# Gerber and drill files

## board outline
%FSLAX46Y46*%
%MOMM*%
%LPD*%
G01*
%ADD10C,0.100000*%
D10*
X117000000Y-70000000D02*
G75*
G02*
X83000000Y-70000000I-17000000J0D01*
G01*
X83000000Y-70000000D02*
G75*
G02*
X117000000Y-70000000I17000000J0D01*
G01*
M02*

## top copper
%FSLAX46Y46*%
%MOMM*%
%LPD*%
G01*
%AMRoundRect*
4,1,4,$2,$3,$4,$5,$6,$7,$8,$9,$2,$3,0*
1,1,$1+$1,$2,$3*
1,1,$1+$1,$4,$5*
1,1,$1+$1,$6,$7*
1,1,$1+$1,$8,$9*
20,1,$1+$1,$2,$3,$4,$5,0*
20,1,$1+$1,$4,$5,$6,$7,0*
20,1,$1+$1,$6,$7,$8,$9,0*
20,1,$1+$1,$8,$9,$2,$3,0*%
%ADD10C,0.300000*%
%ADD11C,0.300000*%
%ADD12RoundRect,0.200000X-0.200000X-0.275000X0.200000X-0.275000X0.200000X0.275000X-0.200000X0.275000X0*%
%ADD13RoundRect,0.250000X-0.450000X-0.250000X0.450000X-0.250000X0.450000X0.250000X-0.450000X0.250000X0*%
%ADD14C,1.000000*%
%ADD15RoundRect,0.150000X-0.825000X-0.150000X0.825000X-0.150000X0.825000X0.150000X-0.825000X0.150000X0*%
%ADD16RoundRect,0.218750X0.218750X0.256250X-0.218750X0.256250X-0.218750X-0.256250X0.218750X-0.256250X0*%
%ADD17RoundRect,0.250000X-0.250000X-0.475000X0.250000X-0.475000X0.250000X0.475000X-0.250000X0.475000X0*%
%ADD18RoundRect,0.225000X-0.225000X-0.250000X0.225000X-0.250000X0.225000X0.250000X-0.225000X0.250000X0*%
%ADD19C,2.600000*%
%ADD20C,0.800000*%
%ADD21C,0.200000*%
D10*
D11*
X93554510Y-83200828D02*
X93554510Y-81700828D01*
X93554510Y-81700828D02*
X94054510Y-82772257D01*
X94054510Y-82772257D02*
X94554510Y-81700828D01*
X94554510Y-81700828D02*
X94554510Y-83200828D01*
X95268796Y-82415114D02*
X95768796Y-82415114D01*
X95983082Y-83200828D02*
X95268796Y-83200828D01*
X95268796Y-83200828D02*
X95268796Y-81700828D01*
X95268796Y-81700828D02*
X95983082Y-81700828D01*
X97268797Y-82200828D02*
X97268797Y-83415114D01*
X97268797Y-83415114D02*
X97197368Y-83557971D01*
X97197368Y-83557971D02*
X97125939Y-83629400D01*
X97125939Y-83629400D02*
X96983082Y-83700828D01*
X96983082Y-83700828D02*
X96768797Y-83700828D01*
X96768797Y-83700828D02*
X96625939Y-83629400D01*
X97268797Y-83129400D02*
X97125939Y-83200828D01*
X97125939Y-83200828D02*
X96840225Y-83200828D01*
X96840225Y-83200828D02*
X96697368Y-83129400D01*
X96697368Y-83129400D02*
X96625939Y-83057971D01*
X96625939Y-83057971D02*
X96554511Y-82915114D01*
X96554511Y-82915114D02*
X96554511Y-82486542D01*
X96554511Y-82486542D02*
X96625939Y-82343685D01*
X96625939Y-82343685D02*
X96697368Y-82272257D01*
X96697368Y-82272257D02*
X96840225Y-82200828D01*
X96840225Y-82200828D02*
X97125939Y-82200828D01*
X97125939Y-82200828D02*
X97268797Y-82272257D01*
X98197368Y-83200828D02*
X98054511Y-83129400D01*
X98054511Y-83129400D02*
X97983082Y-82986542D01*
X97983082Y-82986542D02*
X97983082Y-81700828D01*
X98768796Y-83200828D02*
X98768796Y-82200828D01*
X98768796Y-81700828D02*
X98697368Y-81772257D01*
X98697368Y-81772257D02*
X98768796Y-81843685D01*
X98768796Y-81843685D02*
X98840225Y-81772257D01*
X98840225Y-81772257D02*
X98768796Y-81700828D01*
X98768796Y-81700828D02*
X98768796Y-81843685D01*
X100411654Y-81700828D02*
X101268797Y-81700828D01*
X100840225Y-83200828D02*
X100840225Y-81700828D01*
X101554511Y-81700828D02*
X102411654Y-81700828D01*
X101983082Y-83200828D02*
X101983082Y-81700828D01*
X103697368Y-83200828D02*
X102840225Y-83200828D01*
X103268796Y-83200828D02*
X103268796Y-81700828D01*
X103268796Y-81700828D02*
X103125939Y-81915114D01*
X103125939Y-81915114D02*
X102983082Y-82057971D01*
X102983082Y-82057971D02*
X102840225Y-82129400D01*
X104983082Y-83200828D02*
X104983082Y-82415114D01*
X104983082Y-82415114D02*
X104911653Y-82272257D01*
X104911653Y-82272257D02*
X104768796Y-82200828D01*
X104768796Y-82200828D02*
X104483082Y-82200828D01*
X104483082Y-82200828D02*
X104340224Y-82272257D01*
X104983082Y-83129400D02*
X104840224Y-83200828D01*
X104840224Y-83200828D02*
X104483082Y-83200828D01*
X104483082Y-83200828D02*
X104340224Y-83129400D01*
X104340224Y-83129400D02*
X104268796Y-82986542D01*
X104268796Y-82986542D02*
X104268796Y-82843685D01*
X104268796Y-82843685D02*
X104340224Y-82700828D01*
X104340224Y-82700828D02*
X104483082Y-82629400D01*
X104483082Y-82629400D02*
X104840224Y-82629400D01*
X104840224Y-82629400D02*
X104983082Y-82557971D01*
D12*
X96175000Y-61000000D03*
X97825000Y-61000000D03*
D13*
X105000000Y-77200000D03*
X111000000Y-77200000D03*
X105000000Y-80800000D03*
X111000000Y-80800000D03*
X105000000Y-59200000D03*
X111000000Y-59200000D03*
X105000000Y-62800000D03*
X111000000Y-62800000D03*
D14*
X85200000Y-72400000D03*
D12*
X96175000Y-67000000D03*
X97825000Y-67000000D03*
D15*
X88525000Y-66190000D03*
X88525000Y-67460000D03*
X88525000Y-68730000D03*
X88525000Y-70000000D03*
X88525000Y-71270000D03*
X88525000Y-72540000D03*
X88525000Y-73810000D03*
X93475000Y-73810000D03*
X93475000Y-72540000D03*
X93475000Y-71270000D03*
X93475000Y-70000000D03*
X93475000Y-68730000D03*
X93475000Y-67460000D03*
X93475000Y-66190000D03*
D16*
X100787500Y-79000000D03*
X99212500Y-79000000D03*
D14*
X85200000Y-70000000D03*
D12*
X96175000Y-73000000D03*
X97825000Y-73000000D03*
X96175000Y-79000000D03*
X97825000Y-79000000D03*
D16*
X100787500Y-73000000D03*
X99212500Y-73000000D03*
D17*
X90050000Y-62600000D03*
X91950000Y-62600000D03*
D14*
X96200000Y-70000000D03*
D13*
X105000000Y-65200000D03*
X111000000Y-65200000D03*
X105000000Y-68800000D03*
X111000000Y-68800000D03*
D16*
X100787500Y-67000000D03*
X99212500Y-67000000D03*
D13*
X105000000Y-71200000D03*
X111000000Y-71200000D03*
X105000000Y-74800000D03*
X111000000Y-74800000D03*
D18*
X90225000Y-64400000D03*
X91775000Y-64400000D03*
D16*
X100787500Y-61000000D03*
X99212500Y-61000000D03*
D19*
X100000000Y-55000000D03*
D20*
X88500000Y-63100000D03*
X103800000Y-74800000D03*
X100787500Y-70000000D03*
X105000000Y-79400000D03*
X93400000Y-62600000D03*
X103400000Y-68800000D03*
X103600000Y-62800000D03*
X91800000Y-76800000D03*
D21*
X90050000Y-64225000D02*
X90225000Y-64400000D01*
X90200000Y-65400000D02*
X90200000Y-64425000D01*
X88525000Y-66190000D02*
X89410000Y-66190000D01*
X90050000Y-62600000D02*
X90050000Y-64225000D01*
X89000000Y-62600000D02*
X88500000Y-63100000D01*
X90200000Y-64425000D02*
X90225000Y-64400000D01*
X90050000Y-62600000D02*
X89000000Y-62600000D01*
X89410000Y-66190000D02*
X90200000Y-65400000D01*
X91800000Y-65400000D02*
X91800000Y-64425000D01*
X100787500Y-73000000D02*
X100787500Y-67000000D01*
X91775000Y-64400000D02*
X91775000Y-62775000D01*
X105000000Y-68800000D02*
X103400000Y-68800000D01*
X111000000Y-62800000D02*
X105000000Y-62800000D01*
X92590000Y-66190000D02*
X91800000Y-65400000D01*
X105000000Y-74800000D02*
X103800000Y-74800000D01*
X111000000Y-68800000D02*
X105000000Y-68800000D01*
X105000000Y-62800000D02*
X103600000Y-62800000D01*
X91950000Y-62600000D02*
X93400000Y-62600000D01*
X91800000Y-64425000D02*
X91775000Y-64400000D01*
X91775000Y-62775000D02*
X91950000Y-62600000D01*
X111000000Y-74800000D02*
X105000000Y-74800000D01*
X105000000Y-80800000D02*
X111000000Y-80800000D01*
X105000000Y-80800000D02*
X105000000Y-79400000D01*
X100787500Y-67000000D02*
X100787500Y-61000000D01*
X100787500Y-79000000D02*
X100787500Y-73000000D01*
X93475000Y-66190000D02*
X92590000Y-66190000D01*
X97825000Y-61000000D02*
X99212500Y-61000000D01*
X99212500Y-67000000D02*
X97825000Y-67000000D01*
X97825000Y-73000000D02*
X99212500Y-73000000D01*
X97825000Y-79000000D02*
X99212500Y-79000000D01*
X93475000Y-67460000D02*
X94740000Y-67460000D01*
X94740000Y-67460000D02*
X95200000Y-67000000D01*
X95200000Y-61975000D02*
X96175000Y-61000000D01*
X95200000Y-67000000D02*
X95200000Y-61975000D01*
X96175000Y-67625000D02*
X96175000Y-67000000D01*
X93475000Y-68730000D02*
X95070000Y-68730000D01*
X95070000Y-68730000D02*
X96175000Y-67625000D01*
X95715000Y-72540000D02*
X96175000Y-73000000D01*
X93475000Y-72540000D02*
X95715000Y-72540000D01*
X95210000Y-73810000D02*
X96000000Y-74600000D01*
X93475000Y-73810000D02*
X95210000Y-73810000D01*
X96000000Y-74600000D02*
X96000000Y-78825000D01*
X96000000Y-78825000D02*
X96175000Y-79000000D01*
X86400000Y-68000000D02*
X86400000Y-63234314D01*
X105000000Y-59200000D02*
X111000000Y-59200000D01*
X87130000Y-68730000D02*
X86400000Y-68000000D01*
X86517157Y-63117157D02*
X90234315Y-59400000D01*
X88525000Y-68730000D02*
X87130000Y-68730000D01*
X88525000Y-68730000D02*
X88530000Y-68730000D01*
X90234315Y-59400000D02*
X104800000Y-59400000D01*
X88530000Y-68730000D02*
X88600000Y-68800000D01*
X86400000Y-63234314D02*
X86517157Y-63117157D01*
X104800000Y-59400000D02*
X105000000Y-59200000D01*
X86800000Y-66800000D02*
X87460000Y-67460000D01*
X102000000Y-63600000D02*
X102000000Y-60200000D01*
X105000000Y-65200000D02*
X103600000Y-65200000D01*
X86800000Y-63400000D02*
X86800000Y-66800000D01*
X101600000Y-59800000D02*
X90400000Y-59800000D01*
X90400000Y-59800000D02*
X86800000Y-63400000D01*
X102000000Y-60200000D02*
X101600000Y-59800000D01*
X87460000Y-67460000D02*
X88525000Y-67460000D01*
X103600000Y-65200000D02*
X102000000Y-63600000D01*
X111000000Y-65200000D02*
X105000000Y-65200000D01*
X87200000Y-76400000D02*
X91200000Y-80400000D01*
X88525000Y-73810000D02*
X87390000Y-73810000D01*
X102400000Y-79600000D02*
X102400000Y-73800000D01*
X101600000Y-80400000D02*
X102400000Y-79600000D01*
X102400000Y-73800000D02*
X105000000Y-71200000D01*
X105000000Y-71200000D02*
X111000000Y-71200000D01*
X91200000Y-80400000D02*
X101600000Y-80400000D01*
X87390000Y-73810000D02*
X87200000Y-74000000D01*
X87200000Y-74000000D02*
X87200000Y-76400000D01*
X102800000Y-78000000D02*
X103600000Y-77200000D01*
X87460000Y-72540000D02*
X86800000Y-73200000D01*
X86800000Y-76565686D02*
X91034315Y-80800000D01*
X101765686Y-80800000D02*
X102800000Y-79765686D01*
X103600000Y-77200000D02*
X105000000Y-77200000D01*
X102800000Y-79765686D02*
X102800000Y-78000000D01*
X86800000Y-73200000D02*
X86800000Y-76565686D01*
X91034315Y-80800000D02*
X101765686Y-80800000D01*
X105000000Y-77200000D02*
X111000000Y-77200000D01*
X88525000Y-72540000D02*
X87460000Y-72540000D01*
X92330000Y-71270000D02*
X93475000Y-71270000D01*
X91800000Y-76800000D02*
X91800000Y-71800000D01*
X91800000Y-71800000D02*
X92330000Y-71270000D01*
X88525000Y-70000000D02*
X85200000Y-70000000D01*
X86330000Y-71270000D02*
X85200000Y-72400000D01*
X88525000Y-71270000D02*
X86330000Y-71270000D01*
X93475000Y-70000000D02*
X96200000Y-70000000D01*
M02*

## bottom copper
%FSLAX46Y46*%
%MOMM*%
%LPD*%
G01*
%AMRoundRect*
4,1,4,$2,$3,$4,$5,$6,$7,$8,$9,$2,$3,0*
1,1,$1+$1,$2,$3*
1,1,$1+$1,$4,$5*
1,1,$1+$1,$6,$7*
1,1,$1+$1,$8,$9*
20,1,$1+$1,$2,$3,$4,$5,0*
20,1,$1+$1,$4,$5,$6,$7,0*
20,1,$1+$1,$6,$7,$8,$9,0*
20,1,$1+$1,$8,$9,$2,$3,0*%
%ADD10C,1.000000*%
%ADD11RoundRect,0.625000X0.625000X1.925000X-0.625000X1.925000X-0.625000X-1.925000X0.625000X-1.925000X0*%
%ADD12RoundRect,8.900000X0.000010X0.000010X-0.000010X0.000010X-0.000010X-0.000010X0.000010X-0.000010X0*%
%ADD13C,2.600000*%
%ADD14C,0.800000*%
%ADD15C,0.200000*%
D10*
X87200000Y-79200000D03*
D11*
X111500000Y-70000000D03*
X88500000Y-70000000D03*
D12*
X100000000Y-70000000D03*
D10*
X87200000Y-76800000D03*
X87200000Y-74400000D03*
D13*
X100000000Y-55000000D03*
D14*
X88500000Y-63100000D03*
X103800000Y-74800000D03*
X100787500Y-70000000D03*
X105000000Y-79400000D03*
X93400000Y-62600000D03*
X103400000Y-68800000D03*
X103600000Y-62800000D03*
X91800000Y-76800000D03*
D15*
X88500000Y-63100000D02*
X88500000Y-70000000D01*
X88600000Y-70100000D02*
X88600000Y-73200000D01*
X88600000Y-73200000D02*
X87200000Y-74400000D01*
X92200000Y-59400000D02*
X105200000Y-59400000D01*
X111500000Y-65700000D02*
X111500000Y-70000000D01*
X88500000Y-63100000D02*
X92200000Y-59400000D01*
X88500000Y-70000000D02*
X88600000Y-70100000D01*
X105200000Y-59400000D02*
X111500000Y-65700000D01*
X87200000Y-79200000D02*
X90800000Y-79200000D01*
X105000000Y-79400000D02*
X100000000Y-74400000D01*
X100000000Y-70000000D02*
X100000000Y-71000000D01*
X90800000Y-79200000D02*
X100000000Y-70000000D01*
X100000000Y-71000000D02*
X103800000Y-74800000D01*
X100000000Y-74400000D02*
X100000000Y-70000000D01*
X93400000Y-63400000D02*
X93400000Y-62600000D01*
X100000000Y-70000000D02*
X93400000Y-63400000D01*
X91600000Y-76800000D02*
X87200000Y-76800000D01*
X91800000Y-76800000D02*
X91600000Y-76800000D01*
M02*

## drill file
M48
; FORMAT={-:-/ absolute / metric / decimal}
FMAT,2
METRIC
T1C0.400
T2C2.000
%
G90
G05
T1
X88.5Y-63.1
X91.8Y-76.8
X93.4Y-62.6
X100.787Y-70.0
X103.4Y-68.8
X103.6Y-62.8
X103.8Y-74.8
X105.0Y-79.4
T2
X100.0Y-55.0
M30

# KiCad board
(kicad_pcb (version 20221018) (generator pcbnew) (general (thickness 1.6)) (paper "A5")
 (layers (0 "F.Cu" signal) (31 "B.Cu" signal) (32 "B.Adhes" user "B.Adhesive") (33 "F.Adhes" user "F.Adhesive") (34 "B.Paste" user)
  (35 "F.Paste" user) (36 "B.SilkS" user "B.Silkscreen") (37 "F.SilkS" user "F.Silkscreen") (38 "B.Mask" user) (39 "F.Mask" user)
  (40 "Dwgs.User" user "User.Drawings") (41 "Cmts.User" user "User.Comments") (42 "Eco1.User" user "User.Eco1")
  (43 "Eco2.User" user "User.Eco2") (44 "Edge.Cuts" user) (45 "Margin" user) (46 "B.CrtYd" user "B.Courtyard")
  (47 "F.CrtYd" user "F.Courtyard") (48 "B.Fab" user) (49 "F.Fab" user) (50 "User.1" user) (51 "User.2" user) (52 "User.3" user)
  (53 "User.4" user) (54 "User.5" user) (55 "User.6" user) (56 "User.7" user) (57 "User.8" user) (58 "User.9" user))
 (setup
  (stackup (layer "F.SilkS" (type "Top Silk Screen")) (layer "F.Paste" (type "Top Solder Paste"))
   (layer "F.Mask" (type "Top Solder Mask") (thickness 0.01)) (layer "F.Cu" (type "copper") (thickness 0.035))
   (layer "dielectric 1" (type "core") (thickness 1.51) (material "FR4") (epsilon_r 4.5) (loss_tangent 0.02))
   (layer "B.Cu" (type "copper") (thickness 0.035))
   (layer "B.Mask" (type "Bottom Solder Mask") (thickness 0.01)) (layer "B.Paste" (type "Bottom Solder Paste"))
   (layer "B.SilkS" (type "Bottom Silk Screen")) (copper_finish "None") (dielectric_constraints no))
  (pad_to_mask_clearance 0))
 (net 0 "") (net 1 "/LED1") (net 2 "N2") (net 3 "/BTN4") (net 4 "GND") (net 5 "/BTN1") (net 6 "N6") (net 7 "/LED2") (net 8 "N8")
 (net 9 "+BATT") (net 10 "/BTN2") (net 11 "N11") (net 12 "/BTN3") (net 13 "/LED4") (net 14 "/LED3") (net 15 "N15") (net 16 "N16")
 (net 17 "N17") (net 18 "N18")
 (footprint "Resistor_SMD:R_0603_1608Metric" (layer "F.Cu") (at 97 61)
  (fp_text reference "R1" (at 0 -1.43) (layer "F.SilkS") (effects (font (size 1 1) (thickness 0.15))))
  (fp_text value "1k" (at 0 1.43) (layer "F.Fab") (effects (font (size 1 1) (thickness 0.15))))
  (pad "1" smd roundrect (at -0.825 0) (size 0.8 0.95) (layers "F.Cu" "F.Paste" "F.Mask") (roundrect_rratio 0.25) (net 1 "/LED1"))
  (pad "2" smd roundrect (at 0.825 0) (size 0.8 0.95) (layers "F.Cu" "F.Paste" "F.Mask") (roundrect_rratio 0.25) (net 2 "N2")))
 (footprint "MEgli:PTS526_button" (layer "F.Cu") (at 108 79)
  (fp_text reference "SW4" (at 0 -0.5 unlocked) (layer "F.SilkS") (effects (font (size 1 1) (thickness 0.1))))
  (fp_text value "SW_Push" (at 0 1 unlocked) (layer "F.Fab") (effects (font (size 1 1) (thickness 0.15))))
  (pad "1" smd roundrect (at -3 -1.8) (size 1.4 1) (layers "F.Cu" "F.Paste" "F.Mask") (roundrect_rratio 0.25) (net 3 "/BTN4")
   (thermal_bridge_angle 45))
  (pad "1" smd roundrect (at 3 -1.8) (size 1.4 1) (layers "F.Cu" "F.Paste" "F.Mask") (roundrect_rratio 0.25) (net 3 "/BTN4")
   (thermal_bridge_angle 45))
  (pad "2" smd roundrect (at -3 1.8) (size 1.4 1) (layers "F.Cu" "F.Paste" "F.Mask") (roundrect_rratio 0.25) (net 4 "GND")
   (thermal_bridge_angle 45))
  (pad "2" smd roundrect (at 3 1.8) (size 1.4 1) (layers "F.Cu" "F.Paste" "F.Mask") (roundrect_rratio 0.25) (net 4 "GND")
   (thermal_bridge_angle 45)))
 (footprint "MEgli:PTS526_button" (layer "F.Cu") (at 108 61)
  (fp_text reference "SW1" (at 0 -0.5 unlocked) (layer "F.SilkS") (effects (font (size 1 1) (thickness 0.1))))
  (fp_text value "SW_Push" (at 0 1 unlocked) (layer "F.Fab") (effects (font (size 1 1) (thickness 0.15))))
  (pad "1" smd roundrect (at -3 -1.8) (size 1.4 1) (layers "F.Cu" "F.Paste" "F.Mask") (roundrect_rratio 0.25) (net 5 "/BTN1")
   (thermal_bridge_angle 45))
  (pad "1" smd roundrect (at 3 -1.8) (size 1.4 1) (layers "F.Cu" "F.Paste" "F.Mask") (roundrect_rratio 0.25) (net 5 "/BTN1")
   (thermal_bridge_angle 45))
  (pad "2" smd roundrect (at -3 1.8) (size 1.4 1) (layers "F.Cu" "F.Paste" "F.Mask") (roundrect_rratio 0.25) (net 4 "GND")
   (thermal_bridge_angle 45))
  (pad "2" smd roundrect (at 3 1.8) (size 1.4 1) (layers "F.Cu" "F.Paste" "F.Mask") (roundrect_rratio 0.25) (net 4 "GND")
   (thermal_bridge_angle 45)))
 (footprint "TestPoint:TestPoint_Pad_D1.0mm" (layer "F.Cu") (at 85.2 72.4)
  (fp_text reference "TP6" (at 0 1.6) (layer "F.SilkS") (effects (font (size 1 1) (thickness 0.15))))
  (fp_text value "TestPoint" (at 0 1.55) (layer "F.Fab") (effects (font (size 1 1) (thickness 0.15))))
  (pad "1" smd circle (at 0 0) (size 1 1) (layers "F.Cu" "F.Mask") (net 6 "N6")))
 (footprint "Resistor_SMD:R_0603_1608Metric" (layer "F.Cu") (at 97 67)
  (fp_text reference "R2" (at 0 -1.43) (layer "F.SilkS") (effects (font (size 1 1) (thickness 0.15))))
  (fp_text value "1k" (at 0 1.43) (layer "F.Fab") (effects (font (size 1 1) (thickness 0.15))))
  (pad "1" smd roundrect (at -0.825 0) (size 0.8 0.95) (layers "F.Cu" "F.Paste" "F.Mask") (roundrect_rratio 0.25) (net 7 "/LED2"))
  (pad "2" smd roundrect (at 0.825 0) (size 0.8 0.95) (layers "F.Cu" "F.Paste" "F.Mask") (roundrect_rratio 0.25) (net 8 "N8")))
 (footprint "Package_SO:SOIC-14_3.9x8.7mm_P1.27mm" (layer "F.Cu") (at 91 70)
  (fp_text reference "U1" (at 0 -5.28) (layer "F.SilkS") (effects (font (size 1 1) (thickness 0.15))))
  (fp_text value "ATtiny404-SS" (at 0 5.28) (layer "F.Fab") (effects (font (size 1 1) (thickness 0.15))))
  (pad "1" smd roundrect (at -2.475 -3.81) (size 1.95 0.6) (layers "F.Cu" "F.Paste" "F.Mask") (roundrect_rratio 0.25) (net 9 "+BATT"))
  (pad "2" smd roundrect (at -2.475 -2.54) (size 1.95 0.6) (layers "F.Cu" "F.Paste" "F.Mask") (roundrect_rratio 0.25) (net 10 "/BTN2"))
  (pad "3" smd roundrect (at -2.475 -1.27) (size 1.95 0.6) (layers "F.Cu" "F.Paste" "F.Mask") (roundrect_rratio 0.25) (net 5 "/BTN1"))
  (pad "4" smd roundrect (at -2.475 0) (size 1.95 0.6) (layers "F.Cu" "F.Paste" "F.Mask") (roundrect_rratio 0.25) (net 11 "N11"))
  (pad "5" smd roundrect (at -2.475 1.27) (size 1.95 0.6) (layers "F.Cu" "F.Paste" "F.Mask") (roundrect_rratio 0.25) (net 6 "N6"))
  (pad "6" smd roundrect (at -2.475 2.54) (size 1.95 0.6) (layers "F.Cu" "F.Paste" "F.Mask") (roundrect_rratio 0.25) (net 3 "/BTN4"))
  (pad "7" smd roundrect (at -2.475 3.81) (size 1.95 0.6) (layers "F.Cu" "F.Paste" "F.Mask") (roundrect_rratio 0.25) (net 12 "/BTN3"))
  (pad "8" smd roundrect (at 2.475 3.81) (size 1.95 0.6) (layers "F.Cu" "F.Paste" "F.Mask") (roundrect_rratio 0.25) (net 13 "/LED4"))
  (pad "9" smd roundrect (at 2.475 2.54) (size 1.95 0.6) (layers "F.Cu" "F.Paste" "F.Mask") (roundrect_rratio 0.25) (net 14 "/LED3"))
  (pad "10" smd roundrect (at 2.475 1.27) (size 1.95 0.6) (layers "F.Cu" "F.Paste" "F.Mask") (roundrect_rratio 0.25) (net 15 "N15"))
  (pad "11" smd roundrect (at 2.475 0) (size 1.95 0.6) (layers "F.Cu" "F.Paste" "F.Mask") (roundrect_rratio 0.25) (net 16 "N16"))
  (pad "12" smd roundrect (at 2.475 -1.27) (size 1.95 0.6) (layers "F.Cu" "F.Paste" "F.Mask") (roundrect_rratio 0.25) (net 7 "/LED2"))
  (pad "13" smd roundrect (at 2.475 -2.54) (size 1.95 0.6) (layers "F.Cu" "F.Paste" "F.Mask") (roundrect_rratio 0.25) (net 1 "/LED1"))
  (pad "14" smd roundrect (at 2.475 -3.81) (size 1.95 0.6) (layers "F.Cu" "F.Paste" "F.Mask") (roundrect_rratio 0.25) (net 4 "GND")))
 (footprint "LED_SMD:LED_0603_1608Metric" (layer "F.Cu") (at 100 79 180)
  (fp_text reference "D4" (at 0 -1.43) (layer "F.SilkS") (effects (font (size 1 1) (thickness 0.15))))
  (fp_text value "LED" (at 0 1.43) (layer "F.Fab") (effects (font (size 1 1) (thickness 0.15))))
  (pad "1" smd roundrect (at -0.7875 0 180) (size 0.875 0.95) (layers "F.Cu" "F.Paste" "F.Mask") (roundrect_rratio 0.25) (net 4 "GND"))
  (pad "2" smd roundrect (at 0.7875 0 180) (size 0.875 0.95) (layers "F.Cu" "F.Paste" "F.Mask") (roundrect_rratio 0.25) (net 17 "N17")))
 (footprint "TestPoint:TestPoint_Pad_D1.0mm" (layer "F.Cu") (at 85.2 70)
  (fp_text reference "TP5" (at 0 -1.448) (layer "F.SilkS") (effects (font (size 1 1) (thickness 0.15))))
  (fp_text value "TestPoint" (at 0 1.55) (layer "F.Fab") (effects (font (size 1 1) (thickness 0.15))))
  (pad "1" smd circle (at 0 0) (size 1 1) (layers "F.Cu" "F.Mask") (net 11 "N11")))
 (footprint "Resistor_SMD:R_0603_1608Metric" (layer "F.Cu") (at 97 73)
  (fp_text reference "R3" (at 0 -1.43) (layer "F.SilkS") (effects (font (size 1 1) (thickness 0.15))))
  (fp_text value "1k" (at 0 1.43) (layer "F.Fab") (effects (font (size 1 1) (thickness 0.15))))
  (pad "1" smd roundrect (at -0.825 0) (size 0.8 0.95) (layers "F.Cu" "F.Paste" "F.Mask") (roundrect_rratio 0.25) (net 14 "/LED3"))
  (pad "2" smd roundrect (at 0.825 0) (size 0.8 0.95) (layers "F.Cu" "F.Paste" "F.Mask") (roundrect_rratio 0.25) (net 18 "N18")))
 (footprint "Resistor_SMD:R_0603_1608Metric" (layer "F.Cu") (at 97 79)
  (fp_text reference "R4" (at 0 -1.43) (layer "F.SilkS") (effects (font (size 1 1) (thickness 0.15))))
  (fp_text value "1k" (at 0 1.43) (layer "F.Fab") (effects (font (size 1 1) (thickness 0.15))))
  (pad "1" smd roundrect (at -0.825 0) (size 0.8 0.95) (layers "F.Cu" "F.Paste" "F.Mask") (roundrect_rratio 0.25) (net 13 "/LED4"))
  (pad "2" smd roundrect (at 0.825 0) (size 0.8 0.95) (layers "F.Cu" "F.Paste" "F.Mask") (roundrect_rratio 0.25) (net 17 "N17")))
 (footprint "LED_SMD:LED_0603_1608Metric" (layer "F.Cu") (at 100 73 180)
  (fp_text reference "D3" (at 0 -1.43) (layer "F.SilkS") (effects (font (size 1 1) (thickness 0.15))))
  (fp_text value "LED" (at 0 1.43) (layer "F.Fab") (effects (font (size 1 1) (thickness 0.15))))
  (pad "1" smd roundrect (at -0.7875 0 180) (size 0.875 0.95) (layers "F.Cu" "F.Paste" "F.Mask") (roundrect_rratio 0.25) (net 4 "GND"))
  (pad "2" smd roundrect (at 0.7875 0 180) (size 0.875 0.95) (layers "F.Cu" "F.Paste" "F.Mask") (roundrect_rratio 0.25) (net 18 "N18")))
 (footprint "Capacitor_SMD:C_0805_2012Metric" (layer "F.Cu") (at 91 62.6)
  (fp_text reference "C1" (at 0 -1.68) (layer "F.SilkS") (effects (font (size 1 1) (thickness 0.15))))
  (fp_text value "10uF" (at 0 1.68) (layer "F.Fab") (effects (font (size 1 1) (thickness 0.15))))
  (pad "1" smd roundrect (at -0.95 0) (size 1 1.45) (layers "F.Cu" "F.Paste" "F.Mask") (roundrect_rratio 0.25) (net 9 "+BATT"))
  (pad "2" smd roundrect (at 0.95 0) (size 1 1.45) (layers "F.Cu" "F.Paste" "F.Mask") (roundrect_rratio 0.25) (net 4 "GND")))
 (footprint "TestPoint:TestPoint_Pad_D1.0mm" (layer "F.Cu") (at 96.2 70)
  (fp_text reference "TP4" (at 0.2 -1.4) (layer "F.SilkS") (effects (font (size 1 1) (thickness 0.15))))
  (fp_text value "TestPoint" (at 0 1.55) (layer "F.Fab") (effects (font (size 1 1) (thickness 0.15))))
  (pad "1" smd circle (at 0 0) (size 1 1) (layers "F.Cu" "F.Mask") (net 16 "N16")))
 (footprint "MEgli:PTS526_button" (layer "F.Cu") (at 108 67)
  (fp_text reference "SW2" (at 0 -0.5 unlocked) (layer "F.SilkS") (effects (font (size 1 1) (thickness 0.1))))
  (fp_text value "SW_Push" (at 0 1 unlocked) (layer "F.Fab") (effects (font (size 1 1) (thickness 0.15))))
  (pad "1" smd roundrect (at -3 -1.8) (size 1.4 1) (layers "F.Cu" "F.Paste" "F.Mask") (roundrect_rratio 0.25) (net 10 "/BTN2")
   (thermal_bridge_angle 45))
  (pad "1" smd roundrect (at 3 -1.8) (size 1.4 1) (layers "F.Cu" "F.Paste" "F.Mask") (roundrect_rratio 0.25) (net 10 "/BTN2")
   (thermal_bridge_angle 45))
  (pad "2" smd roundrect (at -3 1.8) (size 1.4 1) (layers "F.Cu" "F.Paste" "F.Mask") (roundrect_rratio 0.25) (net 4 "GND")
   (thermal_bridge_angle 45))
  (pad "2" smd roundrect (at 3 1.8) (size 1.4 1) (layers "F.Cu" "F.Paste" "F.Mask") (roundrect_rratio 0.25) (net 4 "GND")
   (thermal_bridge_angle 45)))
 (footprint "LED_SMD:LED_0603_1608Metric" (layer "F.Cu") (at 100 67 180)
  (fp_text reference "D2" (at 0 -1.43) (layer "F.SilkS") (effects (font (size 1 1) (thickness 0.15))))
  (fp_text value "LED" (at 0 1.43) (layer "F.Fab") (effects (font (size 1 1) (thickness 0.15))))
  (pad "1" smd roundrect (at -0.7875 0 180) (size 0.875 0.95) (layers "F.Cu" "F.Paste" "F.Mask") (roundrect_rratio 0.25) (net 4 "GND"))
  (pad "2" smd roundrect (at 0.7875 0 180) (size 0.875 0.95) (layers "F.Cu" "F.Paste" "F.Mask") (roundrect_rratio 0.25) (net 8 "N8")))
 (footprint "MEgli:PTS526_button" (layer "F.Cu") (at 108 73)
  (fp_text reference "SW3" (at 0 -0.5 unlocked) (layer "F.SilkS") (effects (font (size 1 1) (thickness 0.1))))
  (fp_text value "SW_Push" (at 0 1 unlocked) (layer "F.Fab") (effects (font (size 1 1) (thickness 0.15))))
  (pad "1" smd roundrect (at -3 -1.8) (size 1.4 1) (layers "F.Cu" "F.Paste" "F.Mask") (roundrect_rratio 0.25) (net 12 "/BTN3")
   (thermal_bridge_angle 45))
  (pad "1" smd roundrect (at 3 -1.8) (size 1.4 1) (layers "F.Cu" "F.Paste" "F.Mask") (roundrect_rratio 0.25) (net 12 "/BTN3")
   (thermal_bridge_angle 45))
  (pad "2" smd roundrect (at -3 1.8) (size 1.4 1) (layers "F.Cu" "F.Paste" "F.Mask") (roundrect_rratio 0.25) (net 4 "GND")
   (thermal_bridge_angle 45))
  (pad "2" smd roundrect (at 3 1.8) (size 1.4 1) (layers "F.Cu" "F.Paste" "F.Mask") (roundrect_rratio 0.25) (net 4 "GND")
   (thermal_bridge_angle 45)))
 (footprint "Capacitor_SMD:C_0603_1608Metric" (layer "F.Cu") (at 91 64.4)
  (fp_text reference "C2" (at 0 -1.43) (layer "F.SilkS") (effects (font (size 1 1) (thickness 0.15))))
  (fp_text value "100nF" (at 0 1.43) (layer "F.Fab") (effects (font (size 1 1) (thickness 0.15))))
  (pad "1" smd roundrect (at -0.775 0) (size 0.9 0.95) (layers "F.Cu" "F.Paste" "F.Mask") (roundrect_rratio 0.25) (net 9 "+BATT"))
  (pad "2" smd roundrect (at 0.775 0) (size 0.9 0.95) (layers "F.Cu" "F.Paste" "F.Mask") (roundrect_rratio 0.25) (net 4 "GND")))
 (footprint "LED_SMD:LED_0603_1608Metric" (layer "F.Cu") (at 100 61 180)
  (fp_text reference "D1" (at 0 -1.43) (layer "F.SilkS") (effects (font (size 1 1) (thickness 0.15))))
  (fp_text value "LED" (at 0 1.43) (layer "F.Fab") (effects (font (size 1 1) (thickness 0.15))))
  (pad "1" smd roundrect (at -0.7875 0 180) (size 0.875 0.95) (layers "F.Cu" "F.Paste" "F.Mask") (roundrect_rratio 0.25) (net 4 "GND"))
  (pad "2" smd roundrect (at 0.7875 0 180) (size 0.875 0.95) (layers "F.Cu" "F.Paste" "F.Mask") (roundrect_rratio 0.25) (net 2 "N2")))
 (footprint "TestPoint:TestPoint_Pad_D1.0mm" (layer "B.Cu") (at 87.2 79.2 180)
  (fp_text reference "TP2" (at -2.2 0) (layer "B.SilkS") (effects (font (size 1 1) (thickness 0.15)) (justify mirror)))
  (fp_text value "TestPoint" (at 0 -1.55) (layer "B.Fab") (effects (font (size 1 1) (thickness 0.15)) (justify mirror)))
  (pad "1" smd circle (at 0 0 180) (size 1 1) (layers "B.Cu" "B.Mask") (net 4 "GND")))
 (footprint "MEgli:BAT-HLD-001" (layer "B.Cu") (at 100 70 180)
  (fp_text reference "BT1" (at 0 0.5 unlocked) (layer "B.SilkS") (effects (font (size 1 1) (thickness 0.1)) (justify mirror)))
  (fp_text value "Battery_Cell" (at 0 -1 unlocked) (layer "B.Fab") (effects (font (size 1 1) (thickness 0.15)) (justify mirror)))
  (pad "1" smd roundrect (at -11.5 0 180) (size 2.5 5.1) (layers "B.Cu" "B.Paste" "B.Mask") (roundrect_rratio 0.25) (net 9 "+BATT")
   (thermal_bridge_angle 45))
  (pad "1" smd roundrect (at 11.5 0 180) (size 2.5 5.1) (layers "B.Cu" "B.Paste" "B.Mask") (roundrect_rratio 0.25) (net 9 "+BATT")
   (thermal_bridge_angle 45))
  (pad "2" smd roundrect (at 0 0 180) (size 17.8 17.8) (layers "B.Cu" "B.Paste" "B.Mask") (roundrect_rratio 0.5) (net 4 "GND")
   (thermal_bridge_angle 45)))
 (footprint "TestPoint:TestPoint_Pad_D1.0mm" (layer "B.Cu") (at 87.2 76.8 180)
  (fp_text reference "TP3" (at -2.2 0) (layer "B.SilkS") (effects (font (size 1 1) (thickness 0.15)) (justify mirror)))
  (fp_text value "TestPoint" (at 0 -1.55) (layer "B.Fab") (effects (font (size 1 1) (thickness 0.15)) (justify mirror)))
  (pad "1" smd circle (at 0 0 180) (size 1 1) (layers "B.Cu" "B.Mask") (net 15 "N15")))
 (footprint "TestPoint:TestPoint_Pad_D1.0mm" (layer "B.Cu") (at 87.2 74.4 180)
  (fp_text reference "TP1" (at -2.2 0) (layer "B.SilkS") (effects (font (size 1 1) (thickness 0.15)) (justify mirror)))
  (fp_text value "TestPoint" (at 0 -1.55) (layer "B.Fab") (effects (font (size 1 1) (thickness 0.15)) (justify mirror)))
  (pad "1" smd circle (at 0 0 180) (size 1 1) (layers "B.Cu" "B.Mask") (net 9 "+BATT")))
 (gr_circle (center 100 70) (end 117 70) (stroke (width 0.1) (type default)) (fill none) (layer "Edge.Cuts"))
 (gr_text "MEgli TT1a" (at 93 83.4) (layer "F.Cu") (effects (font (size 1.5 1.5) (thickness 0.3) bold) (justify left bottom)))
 (via (at 100 55) (size 2.6) (drill 2) (layers "F.Cu" "B.Cu") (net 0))
 (segment (start 90.05 64.225) (end 90.225 64.4) (width 0.2) (layer "F.Cu") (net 9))
 (segment (start 90.2 65.4) (end 90.2 64.425) (width 0.2) (layer "F.Cu") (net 9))
 (segment (start 88.525 66.19) (end 89.41 66.19) (width 0.2) (layer "F.Cu") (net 9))
 (segment (start 90.05 62.6) (end 90.05 64.225) (width 0.2) (layer "F.Cu") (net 9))
 (segment (start 89 62.6) (end 88.5 63.1) (width 0.2) (layer "F.Cu") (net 9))
 (segment (start 90.2 64.425) (end 90.225 64.4) (width 0.2) (layer "F.Cu") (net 9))
 (segment (start 90.05 62.6) (end 89 62.6) (width 0.2) (layer "F.Cu") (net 9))
 (segment (start 89.41 66.19) (end 90.2 65.4) (width 0.2) (layer "F.Cu") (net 9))
 (via (at 88.5 63.1) (size 0.8) (drill 0.4) (layers "F.Cu" "B.Cu") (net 9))
 (segment (start 88.5 63.1) (end 88.5 70) (width 0.2) (layer "B.Cu") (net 9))
 (segment (start 88.6 70.1) (end 88.6 73.2) (width 0.2) (layer "B.Cu") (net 9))
 (segment (start 88.6 73.2) (end 87.2 74.4) (width 0.2) (layer "B.Cu") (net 9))
 (segment (start 92.2 59.4) (end 105.2 59.4) (width 0.2) (layer "B.Cu") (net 9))
 (segment (start 111.5 65.7) (end 111.5 70) (width 0.2) (layer "B.Cu") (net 9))
 (segment (start 88.5 63.1) (end 92.2 59.4) (width 0.2) (layer "B.Cu") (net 9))
 (segment (start 88.5 70) (end 88.6 70.1) (width 0.2) (layer "B.Cu") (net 9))
 (segment (start 105.2 59.4) (end 111.5 65.7) (width 0.2) (layer "B.Cu") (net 9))
 (segment (start 91.8 65.4) (end 91.8 64.425) (width 0.2) (layer "F.Cu") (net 4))
 (segment (start 100.7875 73) (end 100.7875 67) (width 0.2) (layer "F.Cu") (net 4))
 (segment (start 91.775 64.4) (end 91.775 62.775) (width 0.2) (layer "F.Cu") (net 4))
 (segment (start 105 68.8) (end 103.4 68.8) (width 0.2) (layer "F.Cu") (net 4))
 (segment (start 111 62.8) (end 105 62.8) (width 0.2) (layer "F.Cu") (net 4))
 (segment (start 92.59 66.19) (end 91.8 65.4) (width 0.2) (layer "F.Cu") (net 4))
 (segment (start 105 74.8) (end 103.8 74.8) (width 0.2) (layer "F.Cu") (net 4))
 (segment (start 111 68.8) (end 105 68.8) (width 0.2) (layer "F.Cu") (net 4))
 (segment (start 105 62.8) (end 103.6 62.8) (width 0.2) (layer "F.Cu") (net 4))
 (segment (start 91.95 62.6) (end 93.4 62.6) (width 0.2) (layer "F.Cu") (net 4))
 (segment (start 91.8 64.425) (end 91.775 64.4) (width 0.2) (layer "F.Cu") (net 4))
 (segment (start 91.775 62.775) (end 91.95 62.6) (width 0.2) (layer "F.Cu") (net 4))
 (segment (start 111 74.8) (end 105 74.8) (width 0.2) (layer "F.Cu") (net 4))
 (segment (start 105 80.8) (end 111 80.8) (width 0.2) (layer "F.Cu") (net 4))
 (segment (start 105 80.8) (end 105 79.4) (width 0.2) (layer "F.Cu") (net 4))
 (segment (start 100.7875 67) (end 100.7875 61) (width 0.2) (layer "F.Cu") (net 4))
 (segment (start 100.7875 79) (end 100.7875 73) (width 0.2) (layer "F.Cu") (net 4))
 (segment (start 93.475 66.19) (end 92.59 66.19) (width 0.2) (layer "F.Cu") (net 4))
 (via (at 103.8 74.8) (size 0.8) (drill 0.4) (layers "F.Cu" "B.Cu") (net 4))
 (via (at 100.7875 70) (size 0.8) (drill 0.4) (layers "F.Cu" "B.Cu") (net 4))
 (via (at 105 79.4) (size 0.8) (drill 0.4) (layers "F.Cu" "B.Cu") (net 4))
 (via (at 93.4 62.6) (size 0.8) (drill 0.4) (layers "F.Cu" "B.Cu") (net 4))
 (via (at 103.4 68.8) (size 0.8) (drill 0.4) (layers "F.Cu" "B.Cu") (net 4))
 (via (at 103.6 62.8) (size 0.8) (drill 0.4) (layers "F.Cu" "B.Cu") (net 4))
 (segment (start 87.2 79.2) (end 90.8 79.2) (width 0.2) (layer "B.Cu") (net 4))
 (segment (start 105 79.4) (end 100 74.4) (width 0.2) (layer "B.Cu") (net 4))
 (segment (start 100 70) (end 100 71) (width 0.2) (layer "B.Cu") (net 4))
 (segment (start 90.8 79.2) (end 100 70) (width 0.2) (layer "B.Cu") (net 4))
 (segment (start 100 71) (end 103.8 74.8) (width 0.2) (layer "B.Cu") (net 4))
 (segment (start 100 74.4) (end 100 70) (width 0.2) (layer "B.Cu") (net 4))
 (segment (start 93.4 63.4) (end 93.4 62.6) (width 0.2) (layer "B.Cu") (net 4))
 (segment (start 100 70) (end 93.4 63.4) (width 0.2) (layer "B.Cu") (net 4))
 (segment (start 97.825 61) (end 99.2125 61) (width 0.2) (layer "F.Cu") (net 2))
 (segment (start 99.2125 67) (end 97.825 67) (width 0.2) (layer "F.Cu") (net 8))
 (segment (start 97.825 73) (end 99.2125 73) (width 0.2) (layer "F.Cu") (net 18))
 (segment (start 97.825 79) (end 99.2125 79) (width 0.2) (layer "F.Cu") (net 17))
 (segment (start 93.475 67.46) (end 94.74 67.46) (width 0.2) (layer "F.Cu") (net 1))
 (segment (start 94.74 67.46) (end 95.2 67) (width 0.2) (layer "F.Cu") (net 1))
 (segment (start 95.2 61.975) (end 96.175 61) (width 0.2) (layer "F.Cu") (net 1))
 (segment (start 95.2 67) (end 95.2 61.975) (width 0.2) (layer "F.Cu") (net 1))
 (segment (start 96.175 67.625) (end 96.175 67) (width 0.2) (layer "F.Cu") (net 7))
 (segment (start 93.475 68.73) (end 95.07 68.73) (width 0.2) (layer "F.Cu") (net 7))
 (segment (start 95.07 68.73) (end 96.175 67.625) (width 0.2) (layer "F.Cu") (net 7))
 (segment (start 95.715 72.54) (end 96.175 73) (width 0.2) (layer "F.Cu") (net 14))
 (segment (start 93.475 72.54) (end 95.715 72.54) (width 0.2) (layer "F.Cu") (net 14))
 (segment (start 95.21 73.81) (end 96 74.6) (width 0.2) (layer "F.Cu") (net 13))
 (segment (start 93.475 73.81) (end 95.21 73.81) (width 0.2) (layer "F.Cu") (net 13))
 (segment (start 96 74.6) (end 96 78.825) (width 0.2) (layer "F.Cu") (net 13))
 (segment (start 96 78.825) (end 96.175 79) (width 0.2) (layer "F.Cu") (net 13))
 (segment (start 86.4 68) (end 86.4 63.234314) (width 0.2) (layer "F.Cu") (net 5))
 (segment (start 105 59.2) (end 111 59.2) (width 0.2) (layer "F.Cu") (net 5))
 (segment (start 87.13 68.73) (end 86.4 68) (width 0.2) (layer "F.Cu") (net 5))
 (segment (start 86.517157 63.117157) (end 90.234315 59.4) (width 0.2) (layer "F.Cu") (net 5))
 (segment (start 88.525 68.73) (end 87.13 68.73) (width 0.2) (layer "F.Cu") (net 5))
 (segment (start 88.525 68.73) (end 88.53 68.73) (width 0.2) (layer "F.Cu") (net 5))
 (segment (start 90.234315 59.4) (end 104.8 59.4) (width 0.2) (layer "F.Cu") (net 5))
 (segment (start 88.53 68.73) (end 88.6 68.8) (width 0.2) (layer "F.Cu") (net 5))
 (segment (start 86.4 63.234314) (end 86.517157 63.117157) (width 0.2) (layer "F.Cu") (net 5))
 (segment (start 104.8 59.4) (end 105 59.2) (width 0.2) (layer "F.Cu") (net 5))
 (segment (start 86.8 66.8) (end 87.46 67.46) (width 0.2) (layer "F.Cu") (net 10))
 (segment (start 102 63.6) (end 102 60.2) (width 0.2) (layer "F.Cu") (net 10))
 (segment (start 105 65.2) (end 103.6 65.2) (width 0.2) (layer "F.Cu") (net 10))
 (segment (start 86.8 63.4) (end 86.8 66.8) (width 0.2) (layer "F.Cu") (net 10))
 (segment (start 101.6 59.8) (end 90.4 59.8) (width 0.2) (layer "F.Cu") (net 10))
 (segment (start 90.4 59.8) (end 86.8 63.4) (width 0.2) (layer "F.Cu") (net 10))
 (segment (start 102 60.2) (end 101.6 59.8) (width 0.2) (layer "F.Cu") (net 10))
 (segment (start 87.46 67.46) (end 88.525 67.46) (width 0.2) (layer "F.Cu") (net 10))
 (segment (start 103.6 65.2) (end 102 63.6) (width 0.2) (layer "F.Cu") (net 10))
 (segment (start 111 65.2) (end 105 65.2) (width 0.2) (layer "F.Cu") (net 10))
 (segment (start 87.2 76.4) (end 91.2 80.4) (width 0.2) (layer "F.Cu") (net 12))
 (segment (start 88.525 73.81) (end 87.39 73.81) (width 0.2) (layer "F.Cu") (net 12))
 (segment (start 102.4 79.6) (end 102.4 73.8) (width 0.2) (layer "F.Cu") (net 12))
 (segment (start 101.6 80.4) (end 102.4 79.6) (width 0.2) (layer "F.Cu") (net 12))
 (segment (start 102.4 73.8) (end 105 71.2) (width 0.2) (layer "F.Cu") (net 12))
 (segment (start 105 71.2) (end 111 71.2) (width 0.2) (layer "F.Cu") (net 12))
 (segment (start 91.2 80.4) (end 101.6 80.4) (width 0.2) (layer "F.Cu") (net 12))
 (segment (start 87.39 73.81) (end 87.2 74) (width 0.2) (layer "F.Cu") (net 12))
 (segment (start 87.2 74) (end 87.2 76.4) (width 0.2) (layer "F.Cu") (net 12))
 (segment (start 102.8 78) (end 103.6 77.2) (width 0.2) (layer "F.Cu") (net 3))
 (segment (start 87.46 72.54) (end 86.8 73.2) (width 0.2) (layer "F.Cu") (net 3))
 (segment (start 86.8 76.565686) (end 91.034315 80.8) (width 0.2) (layer "F.Cu") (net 3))
 (segment (start 101.765686 80.8) (end 102.8 79.765686) (width 0.2) (layer "F.Cu") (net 3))
 (segment (start 103.6 77.2) (end 105 77.2) (width 0.2) (layer "F.Cu") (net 3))
 (segment (start 102.8 79.765686) (end 102.8 78) (width 0.2) (layer "F.Cu") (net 3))
 (segment (start 86.8 73.2) (end 86.8 76.565686) (width 0.2) (layer "F.Cu") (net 3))
 (segment (start 91.034315 80.8) (end 101.765686 80.8) (width 0.2) (layer "F.Cu") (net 3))
 (segment (start 105 77.2) (end 111 77.2) (width 0.2) (layer "F.Cu") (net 3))
 (segment (start 88.525 72.54) (end 87.46 72.54) (width 0.2) (layer "F.Cu") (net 3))
 (segment (start 92.33 71.27) (end 93.475 71.27) (width 0.2) (layer "F.Cu") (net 15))
 (segment (start 91.8 76.8) (end 91.8 71.8) (width 0.2) (layer "F.Cu") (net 15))
 (segment (start 91.8 71.8) (end 92.33 71.27) (width 0.2) (layer "F.Cu") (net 15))
 (via (at 91.8 76.8) (size 0.8) (drill 0.4) (layers "F.Cu" "B.Cu") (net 15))
 (segment (start 91.6 76.8) (end 87.2 76.8) (width 0.2) (layer "B.Cu") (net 15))
 (segment (start 91.8 76.8) (end 91.6 76.8) (width 0.2) (layer "B.Cu") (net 15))
 (segment (start 88.525 70) (end 85.2 70) (width 0.2) (layer "F.Cu") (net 11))
 (segment (start 86.33 71.27) (end 85.2 72.4) (width 0.2) (layer "F.Cu") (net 6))
 (segment (start 88.525 71.27) (end 86.33 71.27) (width 0.2) (layer "F.Cu") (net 6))
 (segment (start 93.475 70) (end 96.2 70) (width 0.2) (layer "F.Cu") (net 16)))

